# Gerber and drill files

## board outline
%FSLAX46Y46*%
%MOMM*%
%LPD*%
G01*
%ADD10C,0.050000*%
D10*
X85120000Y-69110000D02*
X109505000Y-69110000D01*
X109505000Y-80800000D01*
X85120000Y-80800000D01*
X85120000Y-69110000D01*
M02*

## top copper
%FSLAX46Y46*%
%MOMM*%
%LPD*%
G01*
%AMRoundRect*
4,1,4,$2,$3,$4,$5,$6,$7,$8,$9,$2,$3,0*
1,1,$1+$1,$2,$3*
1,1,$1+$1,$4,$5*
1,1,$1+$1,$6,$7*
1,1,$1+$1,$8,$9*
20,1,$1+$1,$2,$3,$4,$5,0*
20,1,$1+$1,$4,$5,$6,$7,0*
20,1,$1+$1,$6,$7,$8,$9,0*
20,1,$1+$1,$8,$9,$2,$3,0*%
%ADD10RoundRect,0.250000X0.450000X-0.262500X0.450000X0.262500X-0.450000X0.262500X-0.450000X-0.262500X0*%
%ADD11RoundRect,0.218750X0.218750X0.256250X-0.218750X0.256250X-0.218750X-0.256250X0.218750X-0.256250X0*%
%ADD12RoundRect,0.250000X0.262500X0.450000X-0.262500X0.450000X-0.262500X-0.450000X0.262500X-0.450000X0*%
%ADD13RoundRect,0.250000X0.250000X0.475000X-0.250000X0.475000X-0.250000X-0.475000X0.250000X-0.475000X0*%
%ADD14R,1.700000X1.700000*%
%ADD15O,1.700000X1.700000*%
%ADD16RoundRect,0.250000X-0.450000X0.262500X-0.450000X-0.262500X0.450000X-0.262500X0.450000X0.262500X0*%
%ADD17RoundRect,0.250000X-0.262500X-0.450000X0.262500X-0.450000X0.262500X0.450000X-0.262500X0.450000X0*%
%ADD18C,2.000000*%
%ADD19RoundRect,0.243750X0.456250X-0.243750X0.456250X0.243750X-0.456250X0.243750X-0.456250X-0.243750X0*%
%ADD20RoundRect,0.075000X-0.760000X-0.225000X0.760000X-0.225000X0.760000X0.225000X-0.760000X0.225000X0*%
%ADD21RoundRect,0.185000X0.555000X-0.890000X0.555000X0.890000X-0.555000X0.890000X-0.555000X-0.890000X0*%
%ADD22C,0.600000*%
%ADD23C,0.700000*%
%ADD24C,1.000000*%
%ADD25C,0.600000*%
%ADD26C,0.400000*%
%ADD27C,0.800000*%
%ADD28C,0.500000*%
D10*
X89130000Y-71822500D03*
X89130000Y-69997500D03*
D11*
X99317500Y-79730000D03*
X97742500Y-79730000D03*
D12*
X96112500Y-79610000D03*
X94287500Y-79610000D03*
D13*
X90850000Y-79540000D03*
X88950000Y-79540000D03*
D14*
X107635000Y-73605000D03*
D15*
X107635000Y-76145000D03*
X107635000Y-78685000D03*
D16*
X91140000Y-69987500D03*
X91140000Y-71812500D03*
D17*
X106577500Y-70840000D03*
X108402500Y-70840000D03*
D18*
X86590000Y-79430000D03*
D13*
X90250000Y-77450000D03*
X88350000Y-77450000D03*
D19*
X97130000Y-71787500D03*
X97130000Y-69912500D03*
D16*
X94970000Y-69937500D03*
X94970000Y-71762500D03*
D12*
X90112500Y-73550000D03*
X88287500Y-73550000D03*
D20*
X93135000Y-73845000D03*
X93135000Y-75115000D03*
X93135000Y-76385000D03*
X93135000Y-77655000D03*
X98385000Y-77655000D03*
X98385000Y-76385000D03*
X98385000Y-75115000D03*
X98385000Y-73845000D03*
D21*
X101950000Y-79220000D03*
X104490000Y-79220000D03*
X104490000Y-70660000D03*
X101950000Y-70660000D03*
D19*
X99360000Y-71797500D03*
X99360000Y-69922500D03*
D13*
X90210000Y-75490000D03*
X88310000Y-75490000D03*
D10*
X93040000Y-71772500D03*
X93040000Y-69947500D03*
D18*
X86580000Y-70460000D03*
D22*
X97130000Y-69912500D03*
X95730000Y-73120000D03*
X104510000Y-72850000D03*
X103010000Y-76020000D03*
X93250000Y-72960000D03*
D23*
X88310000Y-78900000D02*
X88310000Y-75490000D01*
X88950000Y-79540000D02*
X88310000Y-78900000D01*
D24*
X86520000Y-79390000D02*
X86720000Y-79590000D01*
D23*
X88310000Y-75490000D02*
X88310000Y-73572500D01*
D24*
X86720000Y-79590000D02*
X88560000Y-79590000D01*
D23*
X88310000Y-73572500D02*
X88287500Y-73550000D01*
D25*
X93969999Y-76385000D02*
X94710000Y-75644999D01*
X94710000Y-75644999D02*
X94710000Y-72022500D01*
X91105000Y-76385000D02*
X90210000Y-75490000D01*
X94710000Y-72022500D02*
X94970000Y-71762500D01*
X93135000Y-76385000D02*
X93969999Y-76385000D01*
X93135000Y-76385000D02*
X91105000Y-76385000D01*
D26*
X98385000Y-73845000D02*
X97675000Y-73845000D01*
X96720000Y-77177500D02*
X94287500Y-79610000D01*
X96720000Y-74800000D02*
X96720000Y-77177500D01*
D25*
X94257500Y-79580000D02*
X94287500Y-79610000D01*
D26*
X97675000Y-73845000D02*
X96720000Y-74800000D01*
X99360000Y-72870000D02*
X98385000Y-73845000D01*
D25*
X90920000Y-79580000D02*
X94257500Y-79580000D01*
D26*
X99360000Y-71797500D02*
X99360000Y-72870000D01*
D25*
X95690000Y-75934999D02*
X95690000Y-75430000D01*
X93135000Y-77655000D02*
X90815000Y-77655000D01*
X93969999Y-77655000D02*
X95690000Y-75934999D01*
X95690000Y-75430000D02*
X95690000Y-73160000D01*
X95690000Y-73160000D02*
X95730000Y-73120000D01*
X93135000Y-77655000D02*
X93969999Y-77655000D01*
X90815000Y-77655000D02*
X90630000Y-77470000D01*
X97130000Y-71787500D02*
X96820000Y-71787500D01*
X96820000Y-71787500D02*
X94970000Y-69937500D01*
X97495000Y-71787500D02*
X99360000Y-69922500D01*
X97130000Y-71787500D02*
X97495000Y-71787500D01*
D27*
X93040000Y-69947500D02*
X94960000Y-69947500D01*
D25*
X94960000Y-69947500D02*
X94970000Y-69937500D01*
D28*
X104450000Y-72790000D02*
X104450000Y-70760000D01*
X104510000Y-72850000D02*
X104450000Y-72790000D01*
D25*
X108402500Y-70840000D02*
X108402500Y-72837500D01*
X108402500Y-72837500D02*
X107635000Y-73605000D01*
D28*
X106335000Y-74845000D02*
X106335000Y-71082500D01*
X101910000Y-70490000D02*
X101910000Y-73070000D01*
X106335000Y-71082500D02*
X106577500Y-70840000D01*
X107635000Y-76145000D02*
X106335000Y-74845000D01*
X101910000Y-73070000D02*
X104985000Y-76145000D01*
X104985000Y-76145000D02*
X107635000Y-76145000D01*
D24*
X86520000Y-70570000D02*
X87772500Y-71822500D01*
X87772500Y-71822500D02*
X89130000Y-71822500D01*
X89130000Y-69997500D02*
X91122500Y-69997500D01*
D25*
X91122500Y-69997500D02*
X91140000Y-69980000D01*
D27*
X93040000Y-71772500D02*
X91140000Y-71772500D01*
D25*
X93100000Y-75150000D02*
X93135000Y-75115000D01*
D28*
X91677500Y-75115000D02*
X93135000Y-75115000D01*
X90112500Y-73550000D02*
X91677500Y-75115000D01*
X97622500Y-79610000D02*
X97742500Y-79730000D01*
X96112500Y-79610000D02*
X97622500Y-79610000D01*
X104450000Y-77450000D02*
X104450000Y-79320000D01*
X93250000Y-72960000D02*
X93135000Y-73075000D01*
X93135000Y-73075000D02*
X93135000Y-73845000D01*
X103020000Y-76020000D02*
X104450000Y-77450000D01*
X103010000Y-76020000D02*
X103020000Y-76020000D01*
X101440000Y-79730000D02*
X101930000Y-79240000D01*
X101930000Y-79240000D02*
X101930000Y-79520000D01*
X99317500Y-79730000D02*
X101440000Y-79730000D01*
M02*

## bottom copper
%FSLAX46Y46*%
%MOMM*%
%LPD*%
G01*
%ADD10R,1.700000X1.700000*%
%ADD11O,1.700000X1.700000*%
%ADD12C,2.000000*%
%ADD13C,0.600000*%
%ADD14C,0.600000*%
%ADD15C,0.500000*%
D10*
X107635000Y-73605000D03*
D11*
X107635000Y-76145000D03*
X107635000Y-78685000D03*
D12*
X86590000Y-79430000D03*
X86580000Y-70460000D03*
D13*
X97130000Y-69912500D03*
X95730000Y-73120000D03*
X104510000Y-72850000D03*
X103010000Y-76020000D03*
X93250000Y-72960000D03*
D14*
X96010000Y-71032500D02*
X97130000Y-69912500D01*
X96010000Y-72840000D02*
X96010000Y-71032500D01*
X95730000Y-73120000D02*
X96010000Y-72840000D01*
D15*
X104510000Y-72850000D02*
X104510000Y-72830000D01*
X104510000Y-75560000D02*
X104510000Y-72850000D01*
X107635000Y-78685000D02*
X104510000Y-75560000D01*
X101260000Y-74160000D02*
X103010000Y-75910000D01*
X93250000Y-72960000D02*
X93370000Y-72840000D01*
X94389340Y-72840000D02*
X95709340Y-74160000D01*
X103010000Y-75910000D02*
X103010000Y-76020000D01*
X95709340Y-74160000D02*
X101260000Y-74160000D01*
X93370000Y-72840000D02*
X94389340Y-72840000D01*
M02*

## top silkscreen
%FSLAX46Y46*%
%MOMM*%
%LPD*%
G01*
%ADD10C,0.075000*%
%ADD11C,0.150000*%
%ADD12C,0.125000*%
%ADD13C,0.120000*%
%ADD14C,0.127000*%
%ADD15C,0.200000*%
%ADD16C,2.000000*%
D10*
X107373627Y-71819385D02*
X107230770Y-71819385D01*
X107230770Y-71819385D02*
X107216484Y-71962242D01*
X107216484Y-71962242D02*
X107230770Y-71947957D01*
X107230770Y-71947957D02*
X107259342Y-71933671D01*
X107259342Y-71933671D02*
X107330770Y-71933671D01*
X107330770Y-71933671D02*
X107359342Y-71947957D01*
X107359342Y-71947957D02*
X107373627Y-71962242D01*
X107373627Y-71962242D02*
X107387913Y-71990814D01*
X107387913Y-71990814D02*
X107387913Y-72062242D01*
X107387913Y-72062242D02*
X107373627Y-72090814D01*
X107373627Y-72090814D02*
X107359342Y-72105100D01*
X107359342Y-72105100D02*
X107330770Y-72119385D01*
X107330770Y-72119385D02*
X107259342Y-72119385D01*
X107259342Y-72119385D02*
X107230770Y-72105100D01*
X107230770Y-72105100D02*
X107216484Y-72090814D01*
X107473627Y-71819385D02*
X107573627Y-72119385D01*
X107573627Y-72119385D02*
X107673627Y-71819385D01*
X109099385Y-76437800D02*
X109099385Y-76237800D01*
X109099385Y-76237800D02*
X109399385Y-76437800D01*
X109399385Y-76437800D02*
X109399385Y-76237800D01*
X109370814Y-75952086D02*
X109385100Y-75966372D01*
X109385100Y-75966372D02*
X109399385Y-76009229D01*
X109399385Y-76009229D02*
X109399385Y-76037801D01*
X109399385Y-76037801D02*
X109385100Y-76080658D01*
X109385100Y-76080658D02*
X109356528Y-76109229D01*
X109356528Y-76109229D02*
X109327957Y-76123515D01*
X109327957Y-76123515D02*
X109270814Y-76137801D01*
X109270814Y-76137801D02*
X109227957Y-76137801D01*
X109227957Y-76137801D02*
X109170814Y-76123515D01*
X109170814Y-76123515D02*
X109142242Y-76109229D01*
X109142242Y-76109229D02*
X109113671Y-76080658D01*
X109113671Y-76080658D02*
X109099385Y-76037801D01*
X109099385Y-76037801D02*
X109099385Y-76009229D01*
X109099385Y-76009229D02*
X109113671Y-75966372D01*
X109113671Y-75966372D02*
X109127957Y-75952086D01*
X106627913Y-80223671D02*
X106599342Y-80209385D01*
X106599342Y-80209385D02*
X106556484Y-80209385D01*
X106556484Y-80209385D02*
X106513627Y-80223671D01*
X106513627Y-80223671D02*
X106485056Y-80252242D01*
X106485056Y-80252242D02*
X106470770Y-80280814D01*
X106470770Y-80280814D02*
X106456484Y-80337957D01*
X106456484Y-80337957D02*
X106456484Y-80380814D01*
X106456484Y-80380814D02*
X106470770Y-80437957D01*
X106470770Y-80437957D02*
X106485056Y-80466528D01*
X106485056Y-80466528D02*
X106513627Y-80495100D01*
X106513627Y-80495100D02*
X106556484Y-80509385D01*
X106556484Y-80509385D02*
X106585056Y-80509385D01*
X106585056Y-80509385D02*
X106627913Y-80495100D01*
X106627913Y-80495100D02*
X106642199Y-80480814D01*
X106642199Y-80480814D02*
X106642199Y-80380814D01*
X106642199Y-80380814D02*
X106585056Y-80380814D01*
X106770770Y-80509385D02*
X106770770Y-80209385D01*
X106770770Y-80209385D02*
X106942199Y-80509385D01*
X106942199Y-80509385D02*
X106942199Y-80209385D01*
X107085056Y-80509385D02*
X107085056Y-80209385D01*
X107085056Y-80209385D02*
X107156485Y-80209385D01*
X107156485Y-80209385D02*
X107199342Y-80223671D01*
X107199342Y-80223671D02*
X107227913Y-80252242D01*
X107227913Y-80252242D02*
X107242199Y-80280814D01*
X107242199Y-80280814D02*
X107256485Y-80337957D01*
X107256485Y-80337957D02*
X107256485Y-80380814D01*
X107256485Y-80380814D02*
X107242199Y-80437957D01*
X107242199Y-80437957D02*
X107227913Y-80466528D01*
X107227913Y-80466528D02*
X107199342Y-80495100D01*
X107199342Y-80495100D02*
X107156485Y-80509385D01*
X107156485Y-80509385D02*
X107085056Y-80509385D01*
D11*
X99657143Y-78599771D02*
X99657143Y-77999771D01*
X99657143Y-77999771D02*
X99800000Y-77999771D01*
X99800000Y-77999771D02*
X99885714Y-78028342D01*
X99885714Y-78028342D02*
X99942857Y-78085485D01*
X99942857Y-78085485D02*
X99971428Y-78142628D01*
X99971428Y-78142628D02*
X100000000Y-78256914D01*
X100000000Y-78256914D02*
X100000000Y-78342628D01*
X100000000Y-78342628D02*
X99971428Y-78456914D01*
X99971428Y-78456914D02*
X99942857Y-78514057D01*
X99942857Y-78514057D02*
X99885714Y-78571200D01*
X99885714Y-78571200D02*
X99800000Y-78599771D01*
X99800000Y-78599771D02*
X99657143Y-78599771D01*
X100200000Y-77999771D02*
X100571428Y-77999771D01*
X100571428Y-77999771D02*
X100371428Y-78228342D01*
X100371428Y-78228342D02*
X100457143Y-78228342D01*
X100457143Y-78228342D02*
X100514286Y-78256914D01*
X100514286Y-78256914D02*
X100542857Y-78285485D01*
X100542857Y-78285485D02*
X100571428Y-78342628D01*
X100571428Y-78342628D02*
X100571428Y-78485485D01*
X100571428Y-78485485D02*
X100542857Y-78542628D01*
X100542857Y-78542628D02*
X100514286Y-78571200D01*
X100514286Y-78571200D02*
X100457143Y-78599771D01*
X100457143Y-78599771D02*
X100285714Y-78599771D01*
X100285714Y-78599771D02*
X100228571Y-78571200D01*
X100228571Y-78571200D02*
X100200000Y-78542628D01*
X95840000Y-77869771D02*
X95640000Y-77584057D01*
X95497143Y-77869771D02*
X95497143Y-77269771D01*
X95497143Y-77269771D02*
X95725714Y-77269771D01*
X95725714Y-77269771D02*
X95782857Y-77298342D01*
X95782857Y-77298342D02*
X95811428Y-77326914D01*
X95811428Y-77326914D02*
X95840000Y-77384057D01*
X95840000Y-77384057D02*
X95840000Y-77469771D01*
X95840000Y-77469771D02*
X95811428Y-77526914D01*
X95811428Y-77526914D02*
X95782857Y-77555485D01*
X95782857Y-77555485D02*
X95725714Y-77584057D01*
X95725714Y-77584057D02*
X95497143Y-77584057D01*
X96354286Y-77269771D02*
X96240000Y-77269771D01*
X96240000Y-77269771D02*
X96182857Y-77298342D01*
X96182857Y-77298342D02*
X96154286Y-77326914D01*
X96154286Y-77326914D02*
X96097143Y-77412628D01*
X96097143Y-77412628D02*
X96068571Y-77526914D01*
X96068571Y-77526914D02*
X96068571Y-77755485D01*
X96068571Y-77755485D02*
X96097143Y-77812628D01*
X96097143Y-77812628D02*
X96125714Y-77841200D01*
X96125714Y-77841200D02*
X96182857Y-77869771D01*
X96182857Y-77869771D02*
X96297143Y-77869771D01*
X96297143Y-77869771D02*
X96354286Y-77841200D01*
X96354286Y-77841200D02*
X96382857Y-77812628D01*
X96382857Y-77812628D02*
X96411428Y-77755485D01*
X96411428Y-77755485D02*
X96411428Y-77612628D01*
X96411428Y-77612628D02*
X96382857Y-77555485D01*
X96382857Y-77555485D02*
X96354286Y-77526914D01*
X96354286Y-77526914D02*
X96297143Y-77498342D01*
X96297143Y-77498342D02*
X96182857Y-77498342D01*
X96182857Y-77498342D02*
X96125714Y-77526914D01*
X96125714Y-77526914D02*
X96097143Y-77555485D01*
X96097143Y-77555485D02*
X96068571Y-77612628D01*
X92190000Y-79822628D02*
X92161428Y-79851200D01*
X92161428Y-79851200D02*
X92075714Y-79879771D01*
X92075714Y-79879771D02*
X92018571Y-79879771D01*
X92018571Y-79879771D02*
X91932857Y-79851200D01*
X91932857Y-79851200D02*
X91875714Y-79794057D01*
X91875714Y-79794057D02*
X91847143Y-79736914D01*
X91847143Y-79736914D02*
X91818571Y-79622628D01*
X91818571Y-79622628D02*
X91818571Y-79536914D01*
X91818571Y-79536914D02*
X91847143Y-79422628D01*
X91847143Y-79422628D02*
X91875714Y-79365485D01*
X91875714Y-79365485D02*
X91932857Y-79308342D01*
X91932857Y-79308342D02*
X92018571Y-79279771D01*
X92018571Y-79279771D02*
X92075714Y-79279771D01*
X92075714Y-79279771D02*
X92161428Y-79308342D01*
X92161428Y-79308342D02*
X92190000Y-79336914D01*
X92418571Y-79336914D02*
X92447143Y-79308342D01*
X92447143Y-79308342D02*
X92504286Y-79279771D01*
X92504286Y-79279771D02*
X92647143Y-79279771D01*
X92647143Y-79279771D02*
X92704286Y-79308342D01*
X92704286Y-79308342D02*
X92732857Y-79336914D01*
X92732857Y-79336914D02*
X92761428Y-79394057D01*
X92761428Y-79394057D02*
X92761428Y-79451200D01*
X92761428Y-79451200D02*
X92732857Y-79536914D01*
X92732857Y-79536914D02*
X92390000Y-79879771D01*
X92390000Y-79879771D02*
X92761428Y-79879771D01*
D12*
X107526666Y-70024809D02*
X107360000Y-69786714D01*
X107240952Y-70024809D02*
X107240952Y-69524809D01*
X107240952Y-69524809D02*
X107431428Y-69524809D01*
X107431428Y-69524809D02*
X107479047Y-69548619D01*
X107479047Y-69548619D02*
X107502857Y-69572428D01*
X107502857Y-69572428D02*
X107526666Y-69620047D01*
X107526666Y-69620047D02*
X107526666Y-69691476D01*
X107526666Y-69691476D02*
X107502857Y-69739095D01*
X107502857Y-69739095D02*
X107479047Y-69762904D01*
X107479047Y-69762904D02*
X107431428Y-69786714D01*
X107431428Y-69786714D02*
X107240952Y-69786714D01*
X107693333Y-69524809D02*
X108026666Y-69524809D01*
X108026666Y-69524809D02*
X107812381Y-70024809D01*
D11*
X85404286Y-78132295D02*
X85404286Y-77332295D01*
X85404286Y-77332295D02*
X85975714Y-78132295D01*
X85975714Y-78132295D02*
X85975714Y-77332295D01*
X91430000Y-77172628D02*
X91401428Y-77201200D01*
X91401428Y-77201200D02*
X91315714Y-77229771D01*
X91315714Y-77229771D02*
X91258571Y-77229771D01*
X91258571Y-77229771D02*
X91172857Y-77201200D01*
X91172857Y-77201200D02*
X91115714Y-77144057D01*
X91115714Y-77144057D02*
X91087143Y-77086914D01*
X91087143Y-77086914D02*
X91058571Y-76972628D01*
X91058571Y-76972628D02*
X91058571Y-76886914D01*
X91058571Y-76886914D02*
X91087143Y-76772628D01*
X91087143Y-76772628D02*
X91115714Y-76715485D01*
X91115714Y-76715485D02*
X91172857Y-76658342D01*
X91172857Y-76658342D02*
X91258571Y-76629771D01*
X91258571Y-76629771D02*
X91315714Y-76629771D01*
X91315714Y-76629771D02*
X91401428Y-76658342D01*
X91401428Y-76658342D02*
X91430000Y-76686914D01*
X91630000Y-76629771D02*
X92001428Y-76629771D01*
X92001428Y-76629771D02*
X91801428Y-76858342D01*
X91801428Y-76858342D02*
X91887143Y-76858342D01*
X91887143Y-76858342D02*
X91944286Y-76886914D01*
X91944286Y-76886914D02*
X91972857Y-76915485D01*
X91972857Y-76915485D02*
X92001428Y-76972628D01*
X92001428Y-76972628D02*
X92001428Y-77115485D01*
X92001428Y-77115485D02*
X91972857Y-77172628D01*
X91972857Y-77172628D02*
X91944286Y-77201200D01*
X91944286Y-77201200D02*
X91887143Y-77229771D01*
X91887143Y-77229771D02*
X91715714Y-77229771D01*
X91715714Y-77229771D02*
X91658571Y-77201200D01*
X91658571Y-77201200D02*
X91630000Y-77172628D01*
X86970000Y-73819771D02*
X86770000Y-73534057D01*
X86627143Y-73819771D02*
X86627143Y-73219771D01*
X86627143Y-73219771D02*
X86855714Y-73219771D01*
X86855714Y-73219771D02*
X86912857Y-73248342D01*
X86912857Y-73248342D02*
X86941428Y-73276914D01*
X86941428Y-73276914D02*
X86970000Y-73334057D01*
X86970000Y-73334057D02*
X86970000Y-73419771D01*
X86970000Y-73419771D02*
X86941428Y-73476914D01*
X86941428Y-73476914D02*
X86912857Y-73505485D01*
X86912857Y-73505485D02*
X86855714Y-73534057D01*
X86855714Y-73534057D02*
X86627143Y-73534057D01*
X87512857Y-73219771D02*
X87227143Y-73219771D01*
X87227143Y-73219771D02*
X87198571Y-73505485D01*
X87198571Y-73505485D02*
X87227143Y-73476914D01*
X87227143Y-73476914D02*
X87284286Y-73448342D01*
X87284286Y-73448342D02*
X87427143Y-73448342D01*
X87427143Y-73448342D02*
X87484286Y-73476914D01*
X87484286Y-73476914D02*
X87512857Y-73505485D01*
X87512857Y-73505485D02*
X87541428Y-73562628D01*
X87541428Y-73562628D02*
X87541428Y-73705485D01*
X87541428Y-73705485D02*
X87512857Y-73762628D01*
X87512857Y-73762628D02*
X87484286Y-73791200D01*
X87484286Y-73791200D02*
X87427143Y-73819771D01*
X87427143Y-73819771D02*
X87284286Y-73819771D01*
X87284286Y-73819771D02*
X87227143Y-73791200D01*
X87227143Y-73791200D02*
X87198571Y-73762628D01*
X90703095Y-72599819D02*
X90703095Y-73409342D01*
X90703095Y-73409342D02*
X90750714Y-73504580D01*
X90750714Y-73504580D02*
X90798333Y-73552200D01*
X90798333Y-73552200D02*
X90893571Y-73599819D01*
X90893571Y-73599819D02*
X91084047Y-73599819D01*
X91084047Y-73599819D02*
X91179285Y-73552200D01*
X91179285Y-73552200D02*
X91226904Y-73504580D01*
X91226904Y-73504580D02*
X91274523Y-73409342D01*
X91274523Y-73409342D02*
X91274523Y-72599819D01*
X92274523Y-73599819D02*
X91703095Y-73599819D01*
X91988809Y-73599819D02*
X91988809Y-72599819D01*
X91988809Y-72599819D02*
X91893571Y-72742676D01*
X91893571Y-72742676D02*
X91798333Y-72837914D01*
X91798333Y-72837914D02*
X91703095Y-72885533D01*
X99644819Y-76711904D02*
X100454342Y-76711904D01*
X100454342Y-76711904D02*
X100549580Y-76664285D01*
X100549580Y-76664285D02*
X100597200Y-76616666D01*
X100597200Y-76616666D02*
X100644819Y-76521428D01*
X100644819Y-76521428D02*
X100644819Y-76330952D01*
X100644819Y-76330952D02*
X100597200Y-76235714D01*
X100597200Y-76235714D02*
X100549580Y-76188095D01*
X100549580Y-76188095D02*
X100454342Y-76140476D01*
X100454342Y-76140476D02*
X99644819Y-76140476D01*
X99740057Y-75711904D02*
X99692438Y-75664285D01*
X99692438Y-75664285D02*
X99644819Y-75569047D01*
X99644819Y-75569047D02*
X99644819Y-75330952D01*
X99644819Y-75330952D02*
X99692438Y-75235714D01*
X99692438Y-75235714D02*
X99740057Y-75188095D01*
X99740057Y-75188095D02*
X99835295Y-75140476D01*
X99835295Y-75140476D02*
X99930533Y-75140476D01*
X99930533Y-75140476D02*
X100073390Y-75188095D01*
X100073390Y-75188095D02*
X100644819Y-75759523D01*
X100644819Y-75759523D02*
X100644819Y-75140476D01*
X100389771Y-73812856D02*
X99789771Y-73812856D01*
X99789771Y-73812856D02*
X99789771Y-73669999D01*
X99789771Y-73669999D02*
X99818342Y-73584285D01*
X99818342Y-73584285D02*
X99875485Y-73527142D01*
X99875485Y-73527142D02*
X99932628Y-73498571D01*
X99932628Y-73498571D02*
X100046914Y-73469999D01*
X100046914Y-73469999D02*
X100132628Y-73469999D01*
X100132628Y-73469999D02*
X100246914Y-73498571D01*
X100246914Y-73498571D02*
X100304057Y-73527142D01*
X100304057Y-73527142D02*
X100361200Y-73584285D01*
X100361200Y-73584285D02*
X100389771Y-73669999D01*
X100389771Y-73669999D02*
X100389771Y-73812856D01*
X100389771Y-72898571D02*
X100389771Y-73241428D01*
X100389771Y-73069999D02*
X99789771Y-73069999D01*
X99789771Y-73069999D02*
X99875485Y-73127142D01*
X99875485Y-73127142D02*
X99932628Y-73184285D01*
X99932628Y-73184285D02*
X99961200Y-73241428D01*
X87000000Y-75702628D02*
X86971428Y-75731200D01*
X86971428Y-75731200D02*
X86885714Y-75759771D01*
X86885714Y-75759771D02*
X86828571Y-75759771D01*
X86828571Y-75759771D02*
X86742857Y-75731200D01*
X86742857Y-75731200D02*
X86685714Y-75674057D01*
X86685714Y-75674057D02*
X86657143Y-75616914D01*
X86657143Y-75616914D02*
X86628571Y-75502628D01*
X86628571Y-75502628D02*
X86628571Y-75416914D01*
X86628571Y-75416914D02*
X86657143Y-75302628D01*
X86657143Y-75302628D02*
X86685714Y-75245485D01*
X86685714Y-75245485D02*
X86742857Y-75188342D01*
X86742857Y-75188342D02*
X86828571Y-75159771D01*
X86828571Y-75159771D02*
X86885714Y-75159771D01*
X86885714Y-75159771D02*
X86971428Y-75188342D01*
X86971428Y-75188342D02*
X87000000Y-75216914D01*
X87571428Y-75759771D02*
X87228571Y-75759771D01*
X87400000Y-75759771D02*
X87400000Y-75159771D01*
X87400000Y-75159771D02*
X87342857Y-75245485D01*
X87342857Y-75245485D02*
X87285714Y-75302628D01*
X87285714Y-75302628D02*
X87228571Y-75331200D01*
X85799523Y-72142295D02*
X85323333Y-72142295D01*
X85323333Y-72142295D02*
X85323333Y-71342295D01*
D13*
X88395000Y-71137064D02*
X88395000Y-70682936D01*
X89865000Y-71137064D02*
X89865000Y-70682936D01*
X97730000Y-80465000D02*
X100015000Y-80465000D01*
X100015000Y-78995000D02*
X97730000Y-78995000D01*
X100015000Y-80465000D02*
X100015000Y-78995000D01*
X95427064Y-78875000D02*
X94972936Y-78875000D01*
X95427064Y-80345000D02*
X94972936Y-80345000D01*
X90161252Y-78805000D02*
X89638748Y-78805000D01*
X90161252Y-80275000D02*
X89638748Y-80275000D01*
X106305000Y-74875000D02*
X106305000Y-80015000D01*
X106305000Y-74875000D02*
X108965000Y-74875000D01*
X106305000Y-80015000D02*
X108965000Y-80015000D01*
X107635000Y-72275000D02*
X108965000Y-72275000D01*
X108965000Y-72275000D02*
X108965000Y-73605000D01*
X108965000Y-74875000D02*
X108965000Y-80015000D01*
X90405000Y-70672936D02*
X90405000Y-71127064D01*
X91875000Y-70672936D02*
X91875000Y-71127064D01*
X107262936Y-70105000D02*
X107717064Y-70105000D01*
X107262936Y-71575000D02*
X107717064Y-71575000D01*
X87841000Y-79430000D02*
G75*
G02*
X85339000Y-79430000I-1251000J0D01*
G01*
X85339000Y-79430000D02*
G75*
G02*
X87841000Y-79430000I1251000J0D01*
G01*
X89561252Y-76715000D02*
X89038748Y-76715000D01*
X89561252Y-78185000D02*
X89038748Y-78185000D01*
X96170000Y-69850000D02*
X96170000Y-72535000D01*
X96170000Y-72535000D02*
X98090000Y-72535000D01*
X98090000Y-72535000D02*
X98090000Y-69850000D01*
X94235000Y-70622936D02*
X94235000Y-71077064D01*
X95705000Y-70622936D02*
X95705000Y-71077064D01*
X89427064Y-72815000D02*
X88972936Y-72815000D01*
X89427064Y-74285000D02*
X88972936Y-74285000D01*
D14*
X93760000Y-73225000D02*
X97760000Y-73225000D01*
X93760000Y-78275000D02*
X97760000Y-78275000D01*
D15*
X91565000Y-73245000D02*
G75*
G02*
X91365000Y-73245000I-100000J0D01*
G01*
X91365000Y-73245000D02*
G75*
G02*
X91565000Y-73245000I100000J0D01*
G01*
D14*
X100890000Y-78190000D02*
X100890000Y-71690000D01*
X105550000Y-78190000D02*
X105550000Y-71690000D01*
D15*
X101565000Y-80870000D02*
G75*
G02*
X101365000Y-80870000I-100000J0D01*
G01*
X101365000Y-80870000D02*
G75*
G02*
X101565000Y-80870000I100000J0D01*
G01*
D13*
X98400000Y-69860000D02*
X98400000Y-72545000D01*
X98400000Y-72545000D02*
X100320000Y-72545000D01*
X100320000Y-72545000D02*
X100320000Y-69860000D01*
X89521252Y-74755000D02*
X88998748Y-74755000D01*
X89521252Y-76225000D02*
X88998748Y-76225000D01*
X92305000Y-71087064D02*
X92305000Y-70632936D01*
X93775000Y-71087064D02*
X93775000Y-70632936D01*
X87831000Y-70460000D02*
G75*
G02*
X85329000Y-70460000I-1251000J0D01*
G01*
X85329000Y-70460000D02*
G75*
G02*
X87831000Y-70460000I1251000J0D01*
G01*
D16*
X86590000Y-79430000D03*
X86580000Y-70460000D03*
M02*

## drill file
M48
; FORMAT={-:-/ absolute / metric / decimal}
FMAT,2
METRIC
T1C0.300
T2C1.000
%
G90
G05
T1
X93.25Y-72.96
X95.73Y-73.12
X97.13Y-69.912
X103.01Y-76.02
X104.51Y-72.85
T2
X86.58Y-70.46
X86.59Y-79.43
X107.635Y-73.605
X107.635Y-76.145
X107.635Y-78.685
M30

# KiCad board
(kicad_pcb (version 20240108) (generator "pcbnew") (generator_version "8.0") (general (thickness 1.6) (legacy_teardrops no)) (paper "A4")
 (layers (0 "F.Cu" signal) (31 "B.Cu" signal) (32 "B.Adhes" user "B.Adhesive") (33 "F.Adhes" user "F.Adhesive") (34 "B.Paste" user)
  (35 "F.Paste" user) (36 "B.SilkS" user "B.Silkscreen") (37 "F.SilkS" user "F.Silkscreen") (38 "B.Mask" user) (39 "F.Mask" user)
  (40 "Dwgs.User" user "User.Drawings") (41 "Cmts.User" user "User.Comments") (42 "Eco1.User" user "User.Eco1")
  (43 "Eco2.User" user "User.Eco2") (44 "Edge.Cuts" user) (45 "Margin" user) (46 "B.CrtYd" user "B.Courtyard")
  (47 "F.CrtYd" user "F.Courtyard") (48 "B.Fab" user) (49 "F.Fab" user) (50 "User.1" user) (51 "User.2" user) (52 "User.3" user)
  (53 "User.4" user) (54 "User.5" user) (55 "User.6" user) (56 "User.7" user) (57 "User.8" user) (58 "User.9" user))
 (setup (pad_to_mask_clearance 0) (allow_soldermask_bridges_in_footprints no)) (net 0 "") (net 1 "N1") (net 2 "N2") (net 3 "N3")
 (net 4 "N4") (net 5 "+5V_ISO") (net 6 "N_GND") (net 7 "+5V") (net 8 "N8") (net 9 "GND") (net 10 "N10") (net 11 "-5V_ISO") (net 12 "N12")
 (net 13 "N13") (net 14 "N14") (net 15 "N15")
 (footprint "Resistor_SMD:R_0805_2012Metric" (layer "F.Cu") (at 89.13 70.91 90)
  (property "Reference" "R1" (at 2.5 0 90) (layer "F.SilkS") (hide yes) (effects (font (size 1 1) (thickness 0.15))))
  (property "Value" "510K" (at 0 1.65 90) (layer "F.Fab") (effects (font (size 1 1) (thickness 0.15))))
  (fp_line (start -0.227064 -0.735) (end 0.227064 -0.735) (stroke (width 0.12) (type solid)) (layer "F.SilkS"))
  (fp_line (start -0.227064 0.735) (end 0.227064 0.735) (stroke (width 0.12) (type solid)) (layer "F.SilkS"))
  (pad "1" smd roundrect (at -0.9125 0 90) (size 1.025 1.4) (layers "F.Cu" "F.Paste" "F.Mask") (roundrect_rratio 0.243902) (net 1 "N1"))
  (pad "2" smd roundrect (at 0.9125 0 90) (size 1.025 1.4) (layers "F.Cu" "F.Paste" "F.Mask") (roundrect_rratio 0.243902) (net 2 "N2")))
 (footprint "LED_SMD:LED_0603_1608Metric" (layer "F.Cu") (at 98.53 79.73 180)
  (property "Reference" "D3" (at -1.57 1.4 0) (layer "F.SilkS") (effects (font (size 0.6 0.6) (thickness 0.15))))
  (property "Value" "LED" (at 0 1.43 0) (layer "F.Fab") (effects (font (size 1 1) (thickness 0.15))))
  (fp_line (start 0.8 -0.735) (end -1.485 -0.735) (stroke (width 0.12) (type solid)) (layer "F.SilkS"))
  (fp_line (start -1.485 0.735) (end 0.8 0.735) (stroke (width 0.12) (type solid)) (layer "F.SilkS"))
  (fp_line (start -1.485 -0.735) (end -1.485 0.735) (stroke (width 0.12) (type solid)) (layer "F.SilkS"))
  (pad "1" smd roundrect (at -0.7875 0 180) (size 0.875 0.95) (layers "F.Cu" "F.Paste" "F.Mask") (roundrect_rratio 0.25) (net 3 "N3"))
  (pad "2" smd roundrect (at 0.7875 0 180) (size 0.875 0.95) (layers "F.Cu" "F.Paste" "F.Mask") (roundrect_rratio 0.25) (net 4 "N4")))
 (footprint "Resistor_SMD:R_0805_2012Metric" (layer "F.Cu") (at 95.2 79.61 180)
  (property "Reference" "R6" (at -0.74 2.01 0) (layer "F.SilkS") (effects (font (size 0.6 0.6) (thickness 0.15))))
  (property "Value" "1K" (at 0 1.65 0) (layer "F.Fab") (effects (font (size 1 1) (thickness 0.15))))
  (fp_line (start -0.227064 0.735) (end 0.227064 0.735) (stroke (width 0.12) (type solid)) (layer "F.SilkS"))
  (fp_line (start -0.227064 -0.735) (end 0.227064 -0.735) (stroke (width 0.12) (type solid)) (layer "F.SilkS"))
  (pad "1" smd roundrect (at -0.9125 0 180) (size 1.025 1.4) (layers "F.Cu" "F.Paste" "F.Mask") (roundrect_rratio 0.243902) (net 4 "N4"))
  (pad "2" smd roundrect (at 0.9125 0 180) (size 1.025 1.4) (layers "F.Cu" "F.Paste" "F.Mask") (roundrect_rratio 0.243902) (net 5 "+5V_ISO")))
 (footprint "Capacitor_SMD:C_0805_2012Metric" (layer "F.Cu") (at 89.9 79.54 180)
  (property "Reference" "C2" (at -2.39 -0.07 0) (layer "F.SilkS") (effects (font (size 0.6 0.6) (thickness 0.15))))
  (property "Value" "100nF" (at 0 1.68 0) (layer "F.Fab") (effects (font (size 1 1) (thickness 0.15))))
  (fp_line (start -0.261252 0.735) (end 0.261252 0.735) (stroke (width 0.12) (type solid)) (layer "F.SilkS"))
  (fp_line (start -0.261252 -0.735) (end 0.261252 -0.735) (stroke (width 0.12) (type solid)) (layer "F.SilkS"))
  (pad "1" smd roundrect (at -0.95 0 180) (size 1 1.45) (layers "F.Cu" "F.Paste" "F.Mask") (roundrect_rratio 0.25) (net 5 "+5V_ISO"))
  (pad "2" smd roundrect (at 0.95 0 180) (size 1 1.45) (layers "F.Cu" "F.Paste" "F.Mask") (roundrect_rratio 0.25) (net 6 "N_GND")))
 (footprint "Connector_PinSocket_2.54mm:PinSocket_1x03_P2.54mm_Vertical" (layer "F.Cu") (at 107.635 73.605)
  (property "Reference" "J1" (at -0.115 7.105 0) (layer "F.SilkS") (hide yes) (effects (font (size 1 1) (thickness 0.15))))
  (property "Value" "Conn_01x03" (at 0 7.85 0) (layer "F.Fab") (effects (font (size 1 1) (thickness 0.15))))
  (fp_line (start -1.33 1.27) (end -1.33 6.41) (stroke (width 0.12) (type solid)) (layer "F.SilkS"))
  (fp_line (start -1.33 1.27) (end 1.33 1.27) (stroke (width 0.12) (type solid)) (layer "F.SilkS"))
  (fp_line (start -1.33 6.41) (end 1.33 6.41) (stroke (width 0.12) (type solid)) (layer "F.SilkS"))
  (fp_line (start 0 -1.33) (end 1.33 -1.33) (stroke (width 0.12) (type solid)) (layer "F.SilkS"))
  (fp_line (start 1.33 -1.33) (end 1.33 0) (stroke (width 0.12) (type solid)) (layer "F.SilkS"))
  (fp_line (start 1.33 1.27) (end 1.33 6.41) (stroke (width 0.12) (type solid)) (layer "F.SilkS"))
  (pad "1" thru_hole rect (at 0 0) (size 1.7 1.7) (drill 1) (layers "*.Cu" "*.Mask") (remove_unused_layers no) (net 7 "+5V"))
  (pad "2" thru_hole oval (at 0 2.54) (size 1.7 1.7) (drill 1) (layers "*.Cu" "*.Mask") (remove_unused_layers no) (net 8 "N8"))
  (pad "3" thru_hole oval (at 0 5.08) (size 1.7 1.7) (drill 1) (layers "*.Cu" "*.Mask") (remove_unused_layers no) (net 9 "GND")))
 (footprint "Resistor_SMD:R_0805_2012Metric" (layer "F.Cu") (at 91.14 70.9 -90)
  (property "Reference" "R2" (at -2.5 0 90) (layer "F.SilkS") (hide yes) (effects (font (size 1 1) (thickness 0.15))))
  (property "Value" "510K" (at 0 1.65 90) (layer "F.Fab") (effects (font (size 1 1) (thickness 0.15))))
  (fp_line (start -0.227064 0.735) (end 0.227064 0.735) (stroke (width 0.12) (type solid)) (layer "F.SilkS"))
  (fp_line (start -0.227064 -0.735) (end 0.227064 -0.735) (stroke (width 0.12) (type solid)) (layer "F.SilkS"))
  (pad "1" smd roundrect (at -0.9125 0 270) (size 1.025 1.4) (layers "F.Cu" "F.Paste" "F.Mask") (roundrect_rratio 0.243902) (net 2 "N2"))
  (pad "2" smd roundrect (at 0.9125 0 270) (size 1.025 1.4) (layers "F.Cu" "F.Paste" "F.Mask") (roundrect_rratio 0.243902) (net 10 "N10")))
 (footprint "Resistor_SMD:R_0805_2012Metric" (layer "F.Cu") (at 107.49 70.84)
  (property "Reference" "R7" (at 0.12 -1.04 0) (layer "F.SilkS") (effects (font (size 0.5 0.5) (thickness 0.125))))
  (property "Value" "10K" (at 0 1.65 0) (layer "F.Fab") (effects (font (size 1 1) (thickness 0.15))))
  (fp_line (start -0.227064 -0.735) (end 0.227064 -0.735) (stroke (width 0.12) (type solid)) (layer "F.SilkS"))
  (fp_line (start -0.227064 0.735) (end 0.227064 0.735) (stroke (width 0.12) (type solid)) (layer "F.SilkS"))
  (pad "1" smd roundrect (at -0.9125 0) (size 1.025 1.4) (layers "F.Cu" "F.Paste" "F.Mask") (roundrect_rratio 0.243902) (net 8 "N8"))
  (pad "2" smd roundrect (at 0.9125 0) (size 1.025 1.4) (layers "F.Cu" "F.Paste" "F.Mask") (roundrect_rratio 0.243902) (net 7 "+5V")))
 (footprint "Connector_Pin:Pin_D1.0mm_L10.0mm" (layer "F.Cu") (at 86.59 79.43)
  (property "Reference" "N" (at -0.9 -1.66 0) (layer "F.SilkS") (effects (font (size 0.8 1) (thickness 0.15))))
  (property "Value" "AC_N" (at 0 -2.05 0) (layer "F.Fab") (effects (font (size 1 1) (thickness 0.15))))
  (fp_circle (center 0 0) (end 1.25 0.05) (stroke (width 0.12) (type solid)) (fill none) (layer "F.SilkS"))
  (pad "1" thru_hole circle (at 0 0) (size 2 2) (drill 1) (layers "*.Cu" "*.Paste" "*.SilkS" "*.Mask" "B.Adhes") (remove_unused_layers no)
   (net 6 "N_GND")))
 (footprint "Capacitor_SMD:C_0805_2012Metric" (layer "F.Cu") (at 89.3 77.45 180)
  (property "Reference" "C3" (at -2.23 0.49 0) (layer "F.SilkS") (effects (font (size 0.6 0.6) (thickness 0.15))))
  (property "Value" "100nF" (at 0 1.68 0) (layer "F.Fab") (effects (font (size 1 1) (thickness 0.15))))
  (fp_line (start -0.261252 0.735) (end 0.261252 0.735) (stroke (width 0.12) (type solid)) (layer "F.SilkS"))
  (fp_line (start -0.261252 -0.735) (end 0.261252 -0.735) (stroke (width 0.12) (type solid)) (layer "F.SilkS"))
  (pad "1" smd roundrect (at -0.95 0 180) (size 1 1.45) (layers "F.Cu" "F.Paste" "F.Mask") (roundrect_rratio 0.25) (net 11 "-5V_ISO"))
  (pad "2" smd roundrect (at 0.95 0 180) (size 1 1.45) (layers "F.Cu" "F.Paste" "F.Mask") (roundrect_rratio 0.25) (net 6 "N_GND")))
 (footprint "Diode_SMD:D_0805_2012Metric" (layer "F.Cu") (at 97.13 70.85 90)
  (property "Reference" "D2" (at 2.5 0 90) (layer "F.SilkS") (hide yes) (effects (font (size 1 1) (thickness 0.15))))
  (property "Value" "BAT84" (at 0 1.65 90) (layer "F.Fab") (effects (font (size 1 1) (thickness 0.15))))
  (fp_line (start 1 -0.96) (end -1.685 -0.96) (stroke (width 0.12) (type solid)) (layer "F.SilkS"))
  (fp_line (start -1.685 -0.96) (end -1.685 0.96) (stroke (width 0.12) (type solid)) (layer "F.SilkS"))
  (fp_line (start -1.685 0.96) (end 1 0.96) (stroke (width 0.12) (type solid)) (layer "F.SilkS"))
  (pad "1" smd roundrect (at -0.9375 0 90) (size 0.975 1.4) (layers "F.Cu" "F.Paste" "F.Mask") (roundrect_rratio 0.25) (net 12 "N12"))
  (pad "2" smd roundrect (at 0.9375 0 90) (size 0.975 1.4) (layers "F.Cu" "F.Paste" "F.Mask") (roundrect_rratio 0.25) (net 11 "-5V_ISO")))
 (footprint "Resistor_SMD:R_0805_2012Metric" (layer "F.Cu") (at 94.97 70.85 -90)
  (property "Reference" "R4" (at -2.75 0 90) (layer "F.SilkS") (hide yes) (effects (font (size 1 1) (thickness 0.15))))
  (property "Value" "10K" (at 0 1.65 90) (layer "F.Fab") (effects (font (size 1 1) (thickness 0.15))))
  (fp_line (start -0.227064 0.735) (end 0.227064 0.735) (stroke (width 0.12) (type solid)) (layer "F.SilkS"))
  (fp_line (start -0.227064 -0.735) (end 0.227064 -0.735) (stroke (width 0.12) (type solid)) (layer "F.SilkS"))
  (pad "1" smd roundrect (at -0.9125 0 270) (size 1.025 1.4) (layers "F.Cu" "F.Paste" "F.Mask") (roundrect_rratio 0.243902) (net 12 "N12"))
  (pad "2" smd roundrect (at 0.9125 0 270) (size 1.025 1.4) (layers "F.Cu" "F.Paste" "F.Mask") (roundrect_rratio 0.243902) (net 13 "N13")))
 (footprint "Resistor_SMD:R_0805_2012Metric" (layer "F.Cu") (at 89.2 73.55 180)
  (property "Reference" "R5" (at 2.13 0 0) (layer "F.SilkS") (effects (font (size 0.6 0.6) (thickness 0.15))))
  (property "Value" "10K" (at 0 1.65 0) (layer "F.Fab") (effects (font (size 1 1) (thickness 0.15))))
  (fp_line (start -0.227064 0.735) (end 0.227064 0.735) (stroke (width 0.12) (type solid)) (layer "F.SilkS"))
  (fp_line (start -0.227064 -0.735) (end 0.227064 -0.735) (stroke (width 0.12) (type solid)) (layer "F.SilkS"))
  (pad "1" smd roundrect (at -0.9125 0 180) (size 1.025 1.4) (layers "F.Cu" "F.Paste" "F.Mask") (roundrect_rratio 0.243902) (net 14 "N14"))
  (pad "2" smd roundrect (at 0.9125 0 180) (size 1.025 1.4) (layers "F.Cu" "F.Paste" "F.Mask") (roundrect_rratio 0.243902) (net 6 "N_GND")))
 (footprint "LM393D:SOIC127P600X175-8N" (layer "F.Cu") (at 95.76 75.75)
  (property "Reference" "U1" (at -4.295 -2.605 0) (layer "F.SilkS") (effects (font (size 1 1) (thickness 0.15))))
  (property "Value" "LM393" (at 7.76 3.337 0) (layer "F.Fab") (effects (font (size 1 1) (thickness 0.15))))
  (fp_line (start -2 -2.525) (end 2 -2.525) (stroke (width 0.127) (type solid)) (layer "F.SilkS"))
  (fp_line (start -2 2.525) (end 2 2.525) (stroke (width 0.127) (type solid)) (layer "F.SilkS"))
  (fp_circle (center -4.295 -2.505) (end -4.195 -2.505) (stroke (width 0.2) (type solid)) (fill none) (layer "F.SilkS"))
  (pad "1" smd roundrect (at -2.625 -1.905) (size 1.67 0.6) (layers "F.Cu" "F.Paste" "F.Mask") (roundrect_rratio 0.125) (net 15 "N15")
   (solder_mask_margin 0.102))
  (pad "2" smd roundrect (at -2.625 -0.635) (size 1.67 0.6) (layers "F.Cu" "F.Paste" "F.Mask") (roundrect_rratio 0.125) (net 14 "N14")
   (solder_mask_margin 0.102))
  (pad "3" smd roundrect (at -2.625 0.635) (size 1.67 0.6) (layers "F.Cu" "F.Paste" "F.Mask") (roundrect_rratio 0.125) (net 13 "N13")
   (solder_mask_margin 0.102))
  (pad "4" smd roundrect (at -2.625 1.905) (size 1.67 0.6) (layers "F.Cu" "F.Paste" "F.Mask") (roundrect_rratio 0.125) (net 11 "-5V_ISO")
   (solder_mask_margin 0.102))
  (pad "5" smd roundrect (at 2.625 1.905) (size 1.67 0.6) (layers "F.Cu" "F.Paste" "F.Mask") (roundrect_rratio 0.125)
   (solder_mask_margin 0.102))
  (pad "6" smd roundrect (at 2.625 0.635) (size 1.67 0.6) (layers "F.Cu" "F.Paste" "F.Mask") (roundrect_rratio 0.125)
   (solder_mask_margin 0.102))
  (pad "7" smd roundrect (at 2.625 -0.635) (size 1.67 0.6) (layers "F.Cu" "F.Paste" "F.Mask") (roundrect_rratio 0.125)
   (solder_mask_margin 0.102))
  (pad "8" smd roundrect (at 2.625 -1.905) (size 1.67 0.6) (layers "F.Cu" "F.Paste" "F.Mask") (roundrect_rratio 0.125) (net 5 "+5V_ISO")
   (solder_mask_margin 0.102)))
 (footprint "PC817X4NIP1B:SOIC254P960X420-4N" (layer "F.Cu") (at 103.22 74.94 90)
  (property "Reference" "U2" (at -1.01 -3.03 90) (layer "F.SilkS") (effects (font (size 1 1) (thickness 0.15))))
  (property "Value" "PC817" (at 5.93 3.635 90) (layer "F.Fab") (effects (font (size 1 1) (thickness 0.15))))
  (fp_line (start -3.25 -2.33) (end 3.25 -2.33) (stroke (width 0.127) (type solid)) (layer "F.SilkS"))
  (fp_line (start -3.25 2.33) (end 3.25 2.33) (stroke (width 0.127) (type solid)) (layer "F.SilkS"))
  (fp_circle (center -5.93 -1.755) (end -5.83 -1.755) (stroke (width 0.2) (type solid)) (fill none) (layer "F.SilkS"))
  (pad "1" smd roundrect (at -4.28 -1.27 90) (size 2.15 1.48) (layers "F.Cu" "F.Paste" "F.Mask") (roundrect_rratio 0.125) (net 3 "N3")
   (solder_mask_margin 0.102))
  (pad "2" smd roundrect (at -4.28 1.27 90) (size 2.15 1.48) (layers "F.Cu" "F.Paste" "F.Mask") (roundrect_rratio 0.125) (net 15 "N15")
   (solder_mask_margin 0.102))
  (pad "3" smd roundrect (at 4.28 1.27 90) (size 2.15 1.48) (layers "F.Cu" "F.Paste" "F.Mask") (roundrect_rratio 0.125) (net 9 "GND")
   (solder_mask_margin 0.102))
  (pad "4" smd roundrect (at 4.28 -1.27 90) (size 2.15 1.48) (layers "F.Cu" "F.Paste" "F.Mask") (roundrect_rratio 0.125) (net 8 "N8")
   (solder_mask_margin 0.102)))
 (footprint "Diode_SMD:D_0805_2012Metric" (layer "F.Cu") (at 99.36 70.86 90)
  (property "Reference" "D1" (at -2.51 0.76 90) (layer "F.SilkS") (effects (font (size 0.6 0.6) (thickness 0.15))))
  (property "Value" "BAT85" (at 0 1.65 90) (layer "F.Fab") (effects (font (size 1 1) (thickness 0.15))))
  (fp_line (start 1 -0.96) (end -1.685 -0.96) (stroke (width 0.12) (type solid)) (layer "F.SilkS"))
  (fp_line (start -1.685 -0.96) (end -1.685 0.96) (stroke (width 0.12) (type solid)) (layer "F.SilkS"))
  (fp_line (start -1.685 0.96) (end 1 0.96) (stroke (width 0.12) (type solid)) (layer "F.SilkS"))
  (pad "1" smd roundrect (at -0.9375 0 90) (size 0.975 1.4) (layers "F.Cu" "F.Paste" "F.Mask") (roundrect_rratio 0.25) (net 5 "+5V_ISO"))
  (pad "2" smd roundrect (at 0.9375 0 90) (size 0.975 1.4) (layers "F.Cu" "F.Paste" "F.Mask") (roundrect_rratio 0.25) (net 12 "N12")))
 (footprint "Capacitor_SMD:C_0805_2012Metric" (layer "F.Cu") (at 89.26 75.49 180)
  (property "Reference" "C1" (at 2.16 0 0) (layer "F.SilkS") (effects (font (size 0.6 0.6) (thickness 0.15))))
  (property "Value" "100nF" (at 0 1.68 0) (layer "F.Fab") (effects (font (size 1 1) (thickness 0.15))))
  (fp_line (start -0.261252 0.735) (end 0.261252 0.735) (stroke (width 0.12) (type solid)) (layer "F.SilkS"))
  (fp_line (start -0.261252 -0.735) (end 0.261252 -0.735) (stroke (width 0.12) (type solid)) (layer "F.SilkS"))
  (pad "1" smd roundrect (at -0.95 0 180) (size 1 1.45) (layers "F.Cu" "F.Paste" "F.Mask") (roundrect_rratio 0.25) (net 13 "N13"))
  (pad "2" smd roundrect (at 0.95 0 180) (size 1 1.45) (layers "F.Cu" "F.Paste" "F.Mask") (roundrect_rratio 0.25) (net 6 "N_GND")))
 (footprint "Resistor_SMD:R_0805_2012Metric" (layer "F.Cu") (at 93.04 70.86 90)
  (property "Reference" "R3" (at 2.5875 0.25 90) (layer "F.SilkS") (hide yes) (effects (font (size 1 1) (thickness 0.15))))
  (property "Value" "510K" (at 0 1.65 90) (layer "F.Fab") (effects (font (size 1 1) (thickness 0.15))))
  (fp_line (start -0.227064 -0.735) (end 0.227064 -0.735) (stroke (width 0.12) (type solid)) (layer "F.SilkS"))
  (fp_line (start -0.227064 0.735) (end 0.227064 0.735) (stroke (width 0.12) (type solid)) (layer "F.SilkS"))
  (pad "1" smd roundrect (at -0.9125 0 90) (size 1.025 1.4) (layers "F.Cu" "F.Paste" "F.Mask") (roundrect_rratio 0.243902) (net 10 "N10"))
  (pad "2" smd roundrect (at 0.9125 0 90) (size 1.025 1.4) (layers "F.Cu" "F.Paste" "F.Mask") (roundrect_rratio 0.243902) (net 12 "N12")))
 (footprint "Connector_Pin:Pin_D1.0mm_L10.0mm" (layer "F.Cu") (at 86.58 70.46)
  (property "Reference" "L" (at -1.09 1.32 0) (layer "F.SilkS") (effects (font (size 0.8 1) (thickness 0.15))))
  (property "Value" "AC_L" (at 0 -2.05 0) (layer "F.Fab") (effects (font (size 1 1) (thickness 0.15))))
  (fp_circle (center 0 0) (end 1.25 0.05) (stroke (width 0.12) (type solid)) (fill none) (layer "F.SilkS"))
  (pad "1" thru_hole circle (at 0 0) (size 2 2) (drill 1) (layers "*.Cu" "*.SilkS" "*.Mask") (remove_unused_layers no) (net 1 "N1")))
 (gr_rect (start 85.12 69.11) (end 109.505 80.8) (stroke (width 0.05) (type default)) (fill none) (layer "Edge.Cuts"))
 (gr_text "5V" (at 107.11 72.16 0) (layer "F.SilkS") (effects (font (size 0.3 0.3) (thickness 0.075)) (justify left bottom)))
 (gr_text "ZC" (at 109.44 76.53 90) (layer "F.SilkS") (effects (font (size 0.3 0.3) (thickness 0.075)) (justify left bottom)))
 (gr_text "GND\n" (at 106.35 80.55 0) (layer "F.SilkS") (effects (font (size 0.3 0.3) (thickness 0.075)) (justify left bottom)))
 (segment (start 88.31 78.9) (end 88.31 75.49) (width 0.7) (layer "F.Cu") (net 6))
 (segment (start 88.95 79.54) (end 88.31 78.9) (width 0.7) (layer "F.Cu") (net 6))
 (segment (start 86.52 79.39) (end 86.72 79.59) (width 1) (layer "F.Cu") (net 6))
 (segment (start 88.31 75.49) (end 88.31 73.5725) (width 0.7) (layer "F.Cu") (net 6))
 (segment (start 86.72 79.59) (end 88.56 79.59) (width 1) (layer "F.Cu") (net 6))
 (segment (start 88.31 73.5725) (end 88.2875 73.55) (width 0.7) (layer "F.Cu") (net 6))
 (segment (start 93.969999 76.385) (end 94.71 75.644999) (width 0.6) (layer "F.Cu") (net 13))
 (segment (start 94.71 75.644999) (end 94.71 72.0225) (width 0.6) (layer "F.Cu") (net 13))
 (segment (start 91.105 76.385) (end 90.21 75.49) (width 0.6) (layer "F.Cu") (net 13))
 (segment (start 94.71 72.0225) (end 94.97 71.7625) (width 0.6) (layer "F.Cu") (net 13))
 (segment (start 93.135 76.385) (end 93.969999 76.385) (width 0.6) (layer "F.Cu") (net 13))
 (segment (start 93.135 76.385) (end 91.105 76.385) (width 0.6) (layer "F.Cu") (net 13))
 (segment (start 98.385 73.845) (end 97.675 73.845) (width 0.4) (layer "F.Cu") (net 5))
 (segment (start 96.72 77.1775) (end 94.2875 79.61) (width 0.4) (layer "F.Cu") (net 5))
 (segment (start 96.72 74.8) (end 96.72 77.1775) (width 0.4) (layer "F.Cu") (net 5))
 (segment (start 94.2575 79.58) (end 94.2875 79.61) (width 0.6) (layer "F.Cu") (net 5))
 (segment (start 97.675 73.845) (end 96.72 74.8) (width 0.4) (layer "F.Cu") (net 5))
 (segment (start 99.36 72.87) (end 98.385 73.845) (width 0.4) (layer "F.Cu") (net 5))
 (segment (start 90.92 79.58) (end 94.2575 79.58) (width 0.6) (layer "F.Cu") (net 5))
 (segment (start 99.36 71.7975) (end 99.36 72.87) (width 0.4) (layer "F.Cu") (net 5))
 (segment (start 95.69 75.934999) (end 95.69 75.43) (width 0.6) (layer "F.Cu") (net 11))
 (segment (start 93.135 77.655) (end 90.815 77.655) (width 0.6) (layer "F.Cu") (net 11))
 (segment (start 93.969999 77.655) (end 95.69 75.934999) (width 0.6) (layer "F.Cu") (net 11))
 (segment (start 95.69 75.43) (end 95.69 73.16) (width 0.6) (layer "F.Cu") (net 11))
 (segment (start 95.69 73.16) (end 95.73 73.12) (width 0.6) (layer "F.Cu") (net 11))
 (segment (start 93.135 77.655) (end 93.969999 77.655) (width 0.6) (layer "F.Cu") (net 11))
 (segment (start 90.815 77.655) (end 90.63 77.47) (width 0.6) (layer "F.Cu") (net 11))
 (via (at 97.13 69.9125) (size 0.6) (drill 0.3) (layers "F.Cu" "B.Cu") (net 11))
 (via (at 95.73 73.12) (size 0.6) (drill 0.3) (layers "F.Cu" "B.Cu") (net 11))
 (segment (start 96.01 71.0325) (end 97.13 69.9125) (width 0.6) (layer "B.Cu") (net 11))
 (segment (start 96.01 72.84) (end 96.01 71.0325) (width 0.6) (layer "B.Cu") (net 11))
 (segment (start 95.73 73.12) (end 96.01 72.84) (width 0.6) (layer "B.Cu") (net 11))
 (segment (start 97.13 71.7875) (end 96.82 71.7875) (width 0.6) (layer "F.Cu") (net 12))
 (segment (start 96.82 71.7875) (end 94.97 69.9375) (width 0.6) (layer "F.Cu") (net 12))
 (segment (start 97.495 71.7875) (end 99.36 69.9225) (width 0.6) (layer "F.Cu") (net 12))
 (segment (start 97.13 71.7875) (end 97.495 71.7875) (width 0.6) (layer "F.Cu") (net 12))
 (segment (start 93.04 69.9475) (end 94.96 69.9475) (width 0.8) (layer "F.Cu") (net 12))
 (segment (start 94.96 69.9475) (end 94.97 69.9375) (width 0.6) (layer "F.Cu") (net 12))
 (segment (start 104.45 72.79) (end 104.45 70.76) (width 0.5) (layer "F.Cu") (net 9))
 (segment (start 104.51 72.85) (end 104.45 72.79) (width 0.5) (layer "F.Cu") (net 9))
 (via (at 104.51 72.85) (size 0.6) (drill 0.3) (layers "F.Cu" "B.Cu") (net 9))
 (segment (start 104.51 72.85) (end 104.51 72.83) (width 0.5) (layer "B.Cu") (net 9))
 (segment (start 104.51 75.56) (end 104.51 72.85) (width 0.5) (layer "B.Cu") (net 9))
 (segment (start 107.635 78.685) (end 104.51 75.56) (width 0.5) (layer "B.Cu") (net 9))
 (segment (start 108.4025 70.84) (end 108.4025 72.8375) (width 0.6) (layer "F.Cu") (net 7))
 (segment (start 108.4025 72.8375) (end 107.635 73.605) (width 0.6) (layer "F.Cu") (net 7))
 (segment (start 106.335 74.845) (end 106.335 71.0825) (width 0.5) (layer "F.Cu") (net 8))
 (segment (start 101.91 70.49) (end 101.91 73.07) (width 0.5) (layer "F.Cu") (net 8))
 (segment (start 106.335 71.0825) (end 106.5775 70.84) (width 0.5) (layer "F.Cu") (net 8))
 (segment (start 107.635 76.145) (end 106.335 74.845) (width 0.5) (layer "F.Cu") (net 8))
 (segment (start 101.91 73.07) (end 104.985 76.145) (width 0.5) (layer "F.Cu") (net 8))
 (segment (start 104.985 76.145) (end 107.635 76.145) (width 0.5) (layer "F.Cu") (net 8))
 (segment (start 86.52 70.57) (end 87.7725 71.8225) (width 1) (layer "F.Cu") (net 1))
 (segment (start 87.7725 71.8225) (end 89.13 71.8225) (width 1) (layer "F.Cu") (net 1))
 (segment (start 89.13 69.9975) (end 91.1225 69.9975) (width 1) (layer "F.Cu") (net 2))
 (segment (start 91.1225 69.9975) (end 91.14 69.98) (width 0.6) (layer "F.Cu") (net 2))
 (segment (start 93.04 71.7725) (end 91.14 71.7725) (width 0.8) (layer "F.Cu") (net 10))
 (segment (start 93.1 75.15) (end 93.135 75.115) (width 0.6) (layer "F.Cu") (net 14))
 (segment (start 91.6775 75.115) (end 93.135 75.115) (width 0.5) (layer "F.Cu") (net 14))
 (segment (start 90.1125 73.55) (end 91.6775 75.115) (width 0.5) (layer "F.Cu") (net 14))
 (segment (start 97.6225 79.61) (end 97.7425 79.73) (width 0.5) (layer "F.Cu") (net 4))
 (segment (start 96.1125 79.61) (end 97.6225 79.61) (width 0.5) (layer "F.Cu") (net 4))
 (segment (start 104.45 77.45) (end 104.45 79.32) (width 0.5) (layer "F.Cu") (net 15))
 (segment (start 93.25 72.96) (end 93.135 73.075) (width 0.5) (layer "F.Cu") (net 15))
 (segment (start 93.135 73.075) (end 93.135 73.845) (width 0.5) (layer "F.Cu") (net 15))
 (segment (start 103.02 76.02) (end 104.45 77.45) (width 0.5) (layer "F.Cu") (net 15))
 (segment (start 103.01 76.02) (end 103.02 76.02) (width 0.5) (layer "F.Cu") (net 15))
 (via (at 103.01 76.02) (size 0.6) (drill 0.3) (layers "F.Cu" "B.Cu") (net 15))
 (via (at 93.25 72.96) (size 0.6) (drill 0.3) (layers "F.Cu" "B.Cu") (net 15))
 (segment (start 101.26 74.16) (end 103.01 75.91) (width 0.5) (layer "B.Cu") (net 15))
 (segment (start 93.25 72.96) (end 93.37 72.84) (width 0.5) (layer "B.Cu") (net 15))
 (segment (start 94.38934 72.84) (end 95.70934 74.16) (width 0.5) (layer "B.Cu") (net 15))
 (segment (start 103.01 75.91) (end 103.01 76.02) (width 0.5) (layer "B.Cu") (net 15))
 (segment (start 95.70934 74.16) (end 101.26 74.16) (width 0.5) (layer "B.Cu") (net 15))
 (segment (start 93.37 72.84) (end 94.38934 72.84) (width 0.5) (layer "B.Cu") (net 15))
 (segment (start 101.44 79.73) (end 101.93 79.24) (width 0.5) (layer "F.Cu") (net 3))
 (segment (start 101.93 79.24) (end 101.93 79.52) (width 0.5) (layer "F.Cu") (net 3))
 (segment (start 99.3175 79.73) (end 101.44 79.73) (width 0.5) (layer "F.Cu") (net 3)))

